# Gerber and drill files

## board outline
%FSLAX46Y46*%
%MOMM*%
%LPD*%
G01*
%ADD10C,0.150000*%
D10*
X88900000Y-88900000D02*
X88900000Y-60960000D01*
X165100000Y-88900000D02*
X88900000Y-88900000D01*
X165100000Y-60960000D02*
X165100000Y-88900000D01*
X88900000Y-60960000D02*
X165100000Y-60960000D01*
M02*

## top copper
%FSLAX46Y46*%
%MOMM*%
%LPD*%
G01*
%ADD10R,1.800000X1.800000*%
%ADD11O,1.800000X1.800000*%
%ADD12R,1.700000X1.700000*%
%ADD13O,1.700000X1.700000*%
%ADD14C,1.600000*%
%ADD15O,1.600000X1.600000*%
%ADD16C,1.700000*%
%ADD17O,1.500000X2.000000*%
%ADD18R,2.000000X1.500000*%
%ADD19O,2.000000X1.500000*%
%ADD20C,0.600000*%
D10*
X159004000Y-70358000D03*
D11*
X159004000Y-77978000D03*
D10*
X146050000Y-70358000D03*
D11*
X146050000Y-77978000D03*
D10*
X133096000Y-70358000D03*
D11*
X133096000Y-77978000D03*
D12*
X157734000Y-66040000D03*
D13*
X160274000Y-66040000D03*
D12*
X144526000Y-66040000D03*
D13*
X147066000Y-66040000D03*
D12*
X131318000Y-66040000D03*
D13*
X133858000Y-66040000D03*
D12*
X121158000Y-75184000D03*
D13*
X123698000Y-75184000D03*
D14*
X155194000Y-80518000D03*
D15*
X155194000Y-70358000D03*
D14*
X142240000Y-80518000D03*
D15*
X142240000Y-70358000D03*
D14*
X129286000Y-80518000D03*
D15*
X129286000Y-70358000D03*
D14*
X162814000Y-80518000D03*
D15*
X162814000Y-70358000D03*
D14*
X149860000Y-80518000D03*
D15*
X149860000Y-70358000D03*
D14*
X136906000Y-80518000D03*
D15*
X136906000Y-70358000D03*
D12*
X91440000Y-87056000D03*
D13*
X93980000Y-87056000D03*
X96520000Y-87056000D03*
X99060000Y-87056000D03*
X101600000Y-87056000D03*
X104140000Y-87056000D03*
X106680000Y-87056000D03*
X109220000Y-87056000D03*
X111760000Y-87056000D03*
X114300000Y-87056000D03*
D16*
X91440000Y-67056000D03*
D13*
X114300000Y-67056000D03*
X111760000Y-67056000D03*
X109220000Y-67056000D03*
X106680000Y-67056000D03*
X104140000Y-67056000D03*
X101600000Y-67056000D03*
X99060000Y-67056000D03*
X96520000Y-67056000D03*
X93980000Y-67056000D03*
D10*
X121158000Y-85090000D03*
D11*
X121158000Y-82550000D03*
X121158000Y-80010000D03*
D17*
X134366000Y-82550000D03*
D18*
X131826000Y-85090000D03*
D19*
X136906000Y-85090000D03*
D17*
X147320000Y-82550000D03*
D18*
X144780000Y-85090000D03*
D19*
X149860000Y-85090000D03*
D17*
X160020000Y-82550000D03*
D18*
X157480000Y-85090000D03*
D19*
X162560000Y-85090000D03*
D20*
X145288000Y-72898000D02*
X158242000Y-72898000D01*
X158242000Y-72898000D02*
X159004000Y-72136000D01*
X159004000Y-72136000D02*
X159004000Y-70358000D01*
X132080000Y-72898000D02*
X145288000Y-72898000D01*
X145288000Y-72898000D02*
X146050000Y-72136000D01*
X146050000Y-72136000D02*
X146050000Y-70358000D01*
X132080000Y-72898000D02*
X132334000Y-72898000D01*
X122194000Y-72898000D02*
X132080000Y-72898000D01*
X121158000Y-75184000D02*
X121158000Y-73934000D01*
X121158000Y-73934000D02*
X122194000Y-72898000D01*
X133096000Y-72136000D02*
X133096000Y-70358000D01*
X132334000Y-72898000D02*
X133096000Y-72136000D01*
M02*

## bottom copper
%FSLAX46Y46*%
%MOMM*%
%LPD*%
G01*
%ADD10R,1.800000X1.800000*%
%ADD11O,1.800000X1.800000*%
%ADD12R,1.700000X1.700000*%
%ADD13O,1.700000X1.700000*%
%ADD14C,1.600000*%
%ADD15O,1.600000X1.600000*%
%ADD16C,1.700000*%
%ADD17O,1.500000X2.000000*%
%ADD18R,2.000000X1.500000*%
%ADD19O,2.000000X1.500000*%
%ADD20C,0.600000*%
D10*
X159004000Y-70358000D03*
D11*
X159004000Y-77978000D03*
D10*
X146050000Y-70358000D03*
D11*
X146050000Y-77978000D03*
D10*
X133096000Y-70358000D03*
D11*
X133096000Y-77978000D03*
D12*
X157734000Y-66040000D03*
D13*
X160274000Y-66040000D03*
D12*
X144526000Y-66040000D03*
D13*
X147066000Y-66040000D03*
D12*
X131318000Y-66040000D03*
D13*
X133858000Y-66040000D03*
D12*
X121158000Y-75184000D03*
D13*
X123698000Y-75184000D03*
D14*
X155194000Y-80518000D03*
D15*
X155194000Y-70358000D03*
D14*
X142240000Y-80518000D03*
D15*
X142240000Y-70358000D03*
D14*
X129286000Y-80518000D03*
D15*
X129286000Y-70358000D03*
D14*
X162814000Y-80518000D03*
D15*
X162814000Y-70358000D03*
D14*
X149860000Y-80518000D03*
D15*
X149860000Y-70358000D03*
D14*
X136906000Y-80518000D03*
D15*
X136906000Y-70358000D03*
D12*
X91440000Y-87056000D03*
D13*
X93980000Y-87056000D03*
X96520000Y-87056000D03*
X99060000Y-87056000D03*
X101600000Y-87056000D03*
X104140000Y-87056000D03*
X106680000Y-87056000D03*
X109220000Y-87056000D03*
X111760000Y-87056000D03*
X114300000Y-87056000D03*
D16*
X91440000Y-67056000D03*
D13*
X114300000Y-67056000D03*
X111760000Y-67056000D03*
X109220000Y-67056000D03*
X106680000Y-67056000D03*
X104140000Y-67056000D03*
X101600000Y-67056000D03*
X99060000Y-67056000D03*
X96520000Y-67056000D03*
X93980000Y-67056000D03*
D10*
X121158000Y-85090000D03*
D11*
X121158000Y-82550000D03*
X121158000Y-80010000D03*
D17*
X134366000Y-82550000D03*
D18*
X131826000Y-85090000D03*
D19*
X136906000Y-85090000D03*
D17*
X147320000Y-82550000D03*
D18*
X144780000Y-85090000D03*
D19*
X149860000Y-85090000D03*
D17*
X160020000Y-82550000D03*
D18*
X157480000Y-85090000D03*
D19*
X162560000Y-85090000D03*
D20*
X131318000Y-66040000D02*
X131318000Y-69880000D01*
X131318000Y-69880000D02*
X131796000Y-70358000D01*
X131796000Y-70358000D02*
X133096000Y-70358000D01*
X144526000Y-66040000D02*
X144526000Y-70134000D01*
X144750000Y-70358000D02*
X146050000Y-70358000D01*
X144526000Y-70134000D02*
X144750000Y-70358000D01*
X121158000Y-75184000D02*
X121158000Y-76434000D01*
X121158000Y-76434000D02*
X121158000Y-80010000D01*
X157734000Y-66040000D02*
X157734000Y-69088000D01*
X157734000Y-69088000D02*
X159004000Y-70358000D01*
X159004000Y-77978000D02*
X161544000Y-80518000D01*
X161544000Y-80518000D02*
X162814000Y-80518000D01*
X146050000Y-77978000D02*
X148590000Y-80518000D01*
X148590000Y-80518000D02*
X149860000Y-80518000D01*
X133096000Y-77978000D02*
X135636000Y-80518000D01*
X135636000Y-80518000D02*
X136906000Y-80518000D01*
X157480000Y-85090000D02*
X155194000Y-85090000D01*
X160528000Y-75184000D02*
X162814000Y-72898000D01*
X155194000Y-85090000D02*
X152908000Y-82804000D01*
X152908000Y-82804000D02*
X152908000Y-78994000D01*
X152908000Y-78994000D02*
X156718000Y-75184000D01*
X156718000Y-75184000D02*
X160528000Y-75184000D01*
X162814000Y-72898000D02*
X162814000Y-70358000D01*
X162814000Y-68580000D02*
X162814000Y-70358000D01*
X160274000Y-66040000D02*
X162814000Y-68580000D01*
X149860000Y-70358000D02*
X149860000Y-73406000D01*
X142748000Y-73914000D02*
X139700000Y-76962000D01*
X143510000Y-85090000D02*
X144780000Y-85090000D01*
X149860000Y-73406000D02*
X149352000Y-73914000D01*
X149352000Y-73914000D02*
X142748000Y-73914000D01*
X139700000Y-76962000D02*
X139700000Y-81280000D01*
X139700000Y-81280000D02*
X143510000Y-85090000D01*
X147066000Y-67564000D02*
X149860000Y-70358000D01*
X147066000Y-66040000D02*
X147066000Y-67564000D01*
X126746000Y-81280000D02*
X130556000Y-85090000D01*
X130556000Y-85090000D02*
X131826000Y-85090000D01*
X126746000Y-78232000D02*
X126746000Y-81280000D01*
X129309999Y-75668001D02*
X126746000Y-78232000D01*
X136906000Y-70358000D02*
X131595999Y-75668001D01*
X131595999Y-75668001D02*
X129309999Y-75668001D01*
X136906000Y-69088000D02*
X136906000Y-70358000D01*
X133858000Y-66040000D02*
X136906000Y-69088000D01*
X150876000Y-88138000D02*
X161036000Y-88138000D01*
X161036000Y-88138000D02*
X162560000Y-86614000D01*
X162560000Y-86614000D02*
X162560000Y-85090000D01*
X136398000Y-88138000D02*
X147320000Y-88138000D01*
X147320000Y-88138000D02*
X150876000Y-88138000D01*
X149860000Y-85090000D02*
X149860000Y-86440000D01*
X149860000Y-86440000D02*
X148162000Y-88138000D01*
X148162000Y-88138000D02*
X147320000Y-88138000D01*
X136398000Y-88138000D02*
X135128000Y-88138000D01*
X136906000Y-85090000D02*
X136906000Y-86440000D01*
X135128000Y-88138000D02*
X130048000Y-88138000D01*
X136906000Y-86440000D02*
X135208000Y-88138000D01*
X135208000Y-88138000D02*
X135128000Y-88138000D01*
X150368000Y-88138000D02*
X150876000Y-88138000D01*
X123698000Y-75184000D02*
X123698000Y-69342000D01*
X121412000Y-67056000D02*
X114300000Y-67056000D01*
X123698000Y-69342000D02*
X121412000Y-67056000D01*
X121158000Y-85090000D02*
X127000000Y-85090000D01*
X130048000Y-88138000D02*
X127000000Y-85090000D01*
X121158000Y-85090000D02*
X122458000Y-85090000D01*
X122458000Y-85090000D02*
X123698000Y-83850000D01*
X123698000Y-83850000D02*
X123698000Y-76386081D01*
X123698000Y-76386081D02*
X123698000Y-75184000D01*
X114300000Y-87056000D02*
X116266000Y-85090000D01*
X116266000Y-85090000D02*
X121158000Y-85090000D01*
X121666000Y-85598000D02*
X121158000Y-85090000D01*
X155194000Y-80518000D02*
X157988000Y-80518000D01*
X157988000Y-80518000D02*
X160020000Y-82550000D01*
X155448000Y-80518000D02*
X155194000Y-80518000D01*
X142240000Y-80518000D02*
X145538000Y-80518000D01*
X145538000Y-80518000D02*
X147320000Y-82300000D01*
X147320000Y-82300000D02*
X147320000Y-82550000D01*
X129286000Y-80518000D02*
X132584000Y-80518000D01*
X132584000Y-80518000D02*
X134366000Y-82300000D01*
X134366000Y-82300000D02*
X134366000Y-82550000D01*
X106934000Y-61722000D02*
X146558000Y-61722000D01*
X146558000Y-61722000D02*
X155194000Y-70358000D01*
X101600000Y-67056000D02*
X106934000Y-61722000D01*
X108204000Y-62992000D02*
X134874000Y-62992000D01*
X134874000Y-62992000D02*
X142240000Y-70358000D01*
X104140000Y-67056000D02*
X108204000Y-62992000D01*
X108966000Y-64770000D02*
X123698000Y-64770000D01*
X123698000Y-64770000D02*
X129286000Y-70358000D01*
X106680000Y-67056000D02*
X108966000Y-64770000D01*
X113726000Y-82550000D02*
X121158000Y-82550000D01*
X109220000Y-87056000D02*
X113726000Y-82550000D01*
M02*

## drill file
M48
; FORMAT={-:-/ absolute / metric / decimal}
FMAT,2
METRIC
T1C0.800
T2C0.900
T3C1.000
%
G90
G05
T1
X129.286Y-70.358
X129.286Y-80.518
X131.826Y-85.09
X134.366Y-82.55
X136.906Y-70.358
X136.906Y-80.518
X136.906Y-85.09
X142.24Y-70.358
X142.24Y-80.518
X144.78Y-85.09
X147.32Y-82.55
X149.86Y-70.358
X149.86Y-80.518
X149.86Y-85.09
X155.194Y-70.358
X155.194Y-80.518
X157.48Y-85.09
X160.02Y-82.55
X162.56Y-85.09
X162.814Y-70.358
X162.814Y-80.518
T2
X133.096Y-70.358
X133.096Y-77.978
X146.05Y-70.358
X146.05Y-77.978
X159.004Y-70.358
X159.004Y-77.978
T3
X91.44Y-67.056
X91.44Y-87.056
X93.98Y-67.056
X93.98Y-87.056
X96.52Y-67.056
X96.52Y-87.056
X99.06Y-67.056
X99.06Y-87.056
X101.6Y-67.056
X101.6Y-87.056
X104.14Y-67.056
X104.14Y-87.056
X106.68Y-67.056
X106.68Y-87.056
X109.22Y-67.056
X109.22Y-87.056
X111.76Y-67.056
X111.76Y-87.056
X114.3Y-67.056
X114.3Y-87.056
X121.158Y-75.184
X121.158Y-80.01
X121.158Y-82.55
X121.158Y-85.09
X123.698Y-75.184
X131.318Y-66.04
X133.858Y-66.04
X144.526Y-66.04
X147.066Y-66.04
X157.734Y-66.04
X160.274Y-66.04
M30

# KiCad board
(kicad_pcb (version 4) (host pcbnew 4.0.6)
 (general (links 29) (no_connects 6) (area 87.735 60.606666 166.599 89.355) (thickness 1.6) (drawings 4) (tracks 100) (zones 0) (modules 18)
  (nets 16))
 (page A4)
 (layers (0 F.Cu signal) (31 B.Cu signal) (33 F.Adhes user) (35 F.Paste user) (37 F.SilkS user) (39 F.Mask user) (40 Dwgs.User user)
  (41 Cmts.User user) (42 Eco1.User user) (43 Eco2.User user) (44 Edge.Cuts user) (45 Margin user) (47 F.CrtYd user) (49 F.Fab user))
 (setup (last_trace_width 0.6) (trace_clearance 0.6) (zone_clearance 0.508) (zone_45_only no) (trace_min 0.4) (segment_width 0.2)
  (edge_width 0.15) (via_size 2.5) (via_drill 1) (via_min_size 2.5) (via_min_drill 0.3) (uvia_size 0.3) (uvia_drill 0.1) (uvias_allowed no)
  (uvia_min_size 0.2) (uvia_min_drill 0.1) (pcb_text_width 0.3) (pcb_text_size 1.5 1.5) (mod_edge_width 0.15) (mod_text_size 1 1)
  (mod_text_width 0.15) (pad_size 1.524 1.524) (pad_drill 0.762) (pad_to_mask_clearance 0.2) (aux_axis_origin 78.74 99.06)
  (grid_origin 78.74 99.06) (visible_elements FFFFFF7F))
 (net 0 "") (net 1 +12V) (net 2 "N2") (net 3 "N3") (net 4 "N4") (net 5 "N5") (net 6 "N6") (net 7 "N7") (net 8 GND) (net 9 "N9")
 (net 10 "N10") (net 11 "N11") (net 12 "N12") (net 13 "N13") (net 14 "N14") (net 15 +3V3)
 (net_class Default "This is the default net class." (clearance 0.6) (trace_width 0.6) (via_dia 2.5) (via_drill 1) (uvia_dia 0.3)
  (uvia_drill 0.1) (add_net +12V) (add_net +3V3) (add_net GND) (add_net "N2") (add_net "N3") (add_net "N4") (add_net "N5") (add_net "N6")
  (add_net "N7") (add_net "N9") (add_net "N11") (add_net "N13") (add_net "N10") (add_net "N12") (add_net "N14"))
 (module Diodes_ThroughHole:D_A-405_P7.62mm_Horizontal (layer F.Cu) (at 159.004 70.358 270)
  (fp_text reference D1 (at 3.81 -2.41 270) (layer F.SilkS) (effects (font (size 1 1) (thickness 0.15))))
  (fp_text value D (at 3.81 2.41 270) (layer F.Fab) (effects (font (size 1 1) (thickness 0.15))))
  (pad 1 thru_hole rect (at 0 0 270) (size 1.8 1.8) (drill 0.9) (layers *.Cu *.Mask) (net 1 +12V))
  (pad 2 thru_hole oval (at 7.62 0 270) (size 1.8 1.8) (drill 0.9) (layers *.Cu *.Mask) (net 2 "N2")))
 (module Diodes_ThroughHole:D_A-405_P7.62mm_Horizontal (layer F.Cu) (at 146.05 70.358 270)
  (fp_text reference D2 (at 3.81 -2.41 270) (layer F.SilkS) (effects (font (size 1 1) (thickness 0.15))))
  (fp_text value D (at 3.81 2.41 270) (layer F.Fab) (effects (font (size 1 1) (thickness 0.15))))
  (pad 1 thru_hole rect (at 0 0 270) (size 1.8 1.8) (drill 0.9) (layers *.Cu *.Mask) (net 1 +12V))
  (pad 2 thru_hole oval (at 7.62 0 270) (size 1.8 1.8) (drill 0.9) (layers *.Cu *.Mask) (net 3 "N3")))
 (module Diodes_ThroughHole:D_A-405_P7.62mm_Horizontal (layer F.Cu) (at 133.096 70.358 270)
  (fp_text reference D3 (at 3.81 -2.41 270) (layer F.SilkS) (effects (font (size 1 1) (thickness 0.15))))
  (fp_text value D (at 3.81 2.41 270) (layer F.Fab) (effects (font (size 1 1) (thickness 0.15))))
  (pad 1 thru_hole rect (at 0 0 270) (size 1.8 1.8) (drill 0.9) (layers *.Cu *.Mask) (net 1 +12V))
  (pad 2 thru_hole oval (at 7.62 0 270) (size 1.8 1.8) (drill 0.9) (layers *.Cu *.Mask) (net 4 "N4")))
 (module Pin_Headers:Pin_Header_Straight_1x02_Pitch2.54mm (layer F.Cu) (at 157.734 66.04 90)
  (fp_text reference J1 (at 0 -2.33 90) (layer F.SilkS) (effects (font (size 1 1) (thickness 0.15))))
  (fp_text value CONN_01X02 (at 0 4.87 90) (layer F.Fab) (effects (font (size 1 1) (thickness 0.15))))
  (pad 1 thru_hole rect (at 0 0 90) (size 1.7 1.7) (drill 1) (layers *.Cu *.Mask) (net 1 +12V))
  (pad 2 thru_hole oval (at 0 2.54 90) (size 1.7 1.7) (drill 1) (layers *.Cu *.Mask) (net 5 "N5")))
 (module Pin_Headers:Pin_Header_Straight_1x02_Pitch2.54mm (layer F.Cu) (at 144.526 66.04 90)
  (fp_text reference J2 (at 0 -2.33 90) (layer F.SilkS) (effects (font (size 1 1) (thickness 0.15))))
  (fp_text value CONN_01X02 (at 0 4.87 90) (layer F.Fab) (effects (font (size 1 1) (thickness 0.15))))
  (pad 1 thru_hole rect (at 0 0 90) (size 1.7 1.7) (drill 1) (layers *.Cu *.Mask) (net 1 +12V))
  (pad 2 thru_hole oval (at 0 2.54 90) (size 1.7 1.7) (drill 1) (layers *.Cu *.Mask) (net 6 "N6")))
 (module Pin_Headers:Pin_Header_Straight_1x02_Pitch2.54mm (layer F.Cu) (at 131.318 66.04 90)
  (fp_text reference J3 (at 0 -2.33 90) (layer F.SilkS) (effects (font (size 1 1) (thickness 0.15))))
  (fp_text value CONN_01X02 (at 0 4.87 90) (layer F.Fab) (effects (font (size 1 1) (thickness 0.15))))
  (pad 1 thru_hole rect (at 0 0 90) (size 1.7 1.7) (drill 1) (layers *.Cu *.Mask) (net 1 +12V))
  (pad 2 thru_hole oval (at 0 2.54 90) (size 1.7 1.7) (drill 1) (layers *.Cu *.Mask) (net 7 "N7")))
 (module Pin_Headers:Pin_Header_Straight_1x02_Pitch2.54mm (layer F.Cu) (at 121.158 75.184 90)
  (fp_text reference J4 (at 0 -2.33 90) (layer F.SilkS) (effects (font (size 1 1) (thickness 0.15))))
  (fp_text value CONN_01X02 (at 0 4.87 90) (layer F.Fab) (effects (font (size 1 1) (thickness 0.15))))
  (pad 1 thru_hole rect (at 0 0 90) (size 1.7 1.7) (drill 1) (layers *.Cu *.Mask) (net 1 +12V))
  (pad 2 thru_hole oval (at 0 2.54 90) (size 1.7 1.7) (drill 1) (layers *.Cu *.Mask) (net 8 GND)))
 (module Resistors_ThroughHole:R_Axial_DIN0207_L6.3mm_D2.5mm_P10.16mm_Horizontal (layer F.Cu) (at 155.194 80.518 90)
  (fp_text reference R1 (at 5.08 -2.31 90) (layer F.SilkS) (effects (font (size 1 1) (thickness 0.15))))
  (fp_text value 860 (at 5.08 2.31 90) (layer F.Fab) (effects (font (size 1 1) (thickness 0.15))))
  (pad 1 thru_hole circle (at 0 0 90) (size 1.6 1.6) (drill 0.8) (layers *.Cu *.Mask) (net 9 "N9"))
  (pad 2 thru_hole oval (at 10.16 0 90) (size 1.6 1.6) (drill 0.8) (layers *.Cu *.Mask) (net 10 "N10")))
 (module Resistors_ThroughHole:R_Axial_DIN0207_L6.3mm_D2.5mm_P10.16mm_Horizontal (layer F.Cu) (at 142.24 80.518 90)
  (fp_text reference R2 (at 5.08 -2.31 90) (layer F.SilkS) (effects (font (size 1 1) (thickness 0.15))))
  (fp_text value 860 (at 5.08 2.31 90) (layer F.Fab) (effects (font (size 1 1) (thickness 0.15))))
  (pad 1 thru_hole circle (at 0 0 90) (size 1.6 1.6) (drill 0.8) (layers *.Cu *.Mask) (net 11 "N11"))
  (pad 2 thru_hole oval (at 10.16 0 90) (size 1.6 1.6) (drill 0.8) (layers *.Cu *.Mask) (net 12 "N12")))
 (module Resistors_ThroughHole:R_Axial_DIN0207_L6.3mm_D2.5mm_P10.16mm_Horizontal (layer F.Cu) (at 129.286 80.518 90)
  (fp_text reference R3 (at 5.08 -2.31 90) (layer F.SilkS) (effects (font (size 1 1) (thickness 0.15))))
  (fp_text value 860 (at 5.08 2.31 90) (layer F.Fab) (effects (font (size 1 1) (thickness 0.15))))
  (pad 1 thru_hole circle (at 0 0 90) (size 1.6 1.6) (drill 0.8) (layers *.Cu *.Mask) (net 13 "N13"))
  (pad 2 thru_hole oval (at 10.16 0 90) (size 1.6 1.6) (drill 0.8) (layers *.Cu *.Mask) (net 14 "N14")))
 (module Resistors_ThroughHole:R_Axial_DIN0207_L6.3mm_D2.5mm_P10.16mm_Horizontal (layer F.Cu) (at 162.814 80.518 90)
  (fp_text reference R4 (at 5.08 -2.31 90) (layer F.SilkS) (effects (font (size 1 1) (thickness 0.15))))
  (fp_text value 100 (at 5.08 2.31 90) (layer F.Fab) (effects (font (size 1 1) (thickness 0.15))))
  (pad 1 thru_hole circle (at 0 0 90) (size 1.6 1.6) (drill 0.8) (layers *.Cu *.Mask) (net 2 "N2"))
  (pad 2 thru_hole oval (at 10.16 0 90) (size 1.6 1.6) (drill 0.8) (layers *.Cu *.Mask) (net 5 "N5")))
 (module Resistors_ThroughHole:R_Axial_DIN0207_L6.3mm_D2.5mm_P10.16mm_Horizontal (layer F.Cu) (at 149.86 80.518 90)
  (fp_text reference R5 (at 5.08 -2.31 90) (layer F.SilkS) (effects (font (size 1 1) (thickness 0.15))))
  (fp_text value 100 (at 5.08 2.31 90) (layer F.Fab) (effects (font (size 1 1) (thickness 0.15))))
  (pad 1 thru_hole circle (at 0 0 90) (size 1.6 1.6) (drill 0.8) (layers *.Cu *.Mask) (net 3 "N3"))
  (pad 2 thru_hole oval (at 10.16 0 90) (size 1.6 1.6) (drill 0.8) (layers *.Cu *.Mask) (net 6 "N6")))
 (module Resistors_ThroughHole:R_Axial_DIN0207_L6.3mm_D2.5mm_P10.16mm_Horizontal (layer F.Cu) (at 136.906 80.518 90)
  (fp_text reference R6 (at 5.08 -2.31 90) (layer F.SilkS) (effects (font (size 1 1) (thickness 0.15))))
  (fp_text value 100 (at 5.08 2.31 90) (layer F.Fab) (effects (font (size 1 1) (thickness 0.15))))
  (pad 1 thru_hole circle (at 0 0 90) (size 1.6 1.6) (drill 0.8) (layers *.Cu *.Mask) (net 4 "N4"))
  (pad 2 thru_hole oval (at 10.16 0 90) (size 1.6 1.6) (drill 0.8) (layers *.Cu *.Mask) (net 7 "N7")))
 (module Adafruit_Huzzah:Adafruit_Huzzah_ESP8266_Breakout (layer F.Cu) (at 91.44 77.056 90)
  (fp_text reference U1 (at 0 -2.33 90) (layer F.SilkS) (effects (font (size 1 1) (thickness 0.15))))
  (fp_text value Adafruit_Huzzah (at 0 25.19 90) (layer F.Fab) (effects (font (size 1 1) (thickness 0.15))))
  (pad 1 thru_hole rect (at -10 0 90) (size 1.7 1.7) (drill 1) (layers *.Cu *.Mask))
  (pad 3 thru_hole oval (at -10 2.54 90) (size 1.7 1.7) (drill 1) (layers *.Cu *.Mask))
  (pad 5 thru_hole oval (at -10 5.08 90) (size 1.7 1.7) (drill 1) (layers *.Cu *.Mask))
  (pad 7 thru_hole oval (at -10 7.62 90) (size 1.7 1.7) (drill 1) (layers *.Cu *.Mask))
  (pad 9 thru_hole oval (at -10 10.16 90) (size 1.7 1.7) (drill 1) (layers *.Cu *.Mask))
  (pad 11 thru_hole oval (at -10 12.7 90) (size 1.7 1.7) (drill 1) (layers *.Cu *.Mask))
  (pad 13 thru_hole oval (at -10 15.24 90) (size 1.7 1.7) (drill 1) (layers *.Cu *.Mask))
  (pad 15 thru_hole oval (at -10 17.78 90) (size 1.7 1.7) (drill 1) (layers *.Cu *.Mask) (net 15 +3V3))
  (pad 17 thru_hole oval (at -10 20.32 90) (size 1.7 1.7) (drill 1) (layers *.Cu *.Mask))
  (pad 19 thru_hole oval (at -10 22.86 90) (size 1.7 1.7) (drill 1) (layers *.Cu *.Mask) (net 8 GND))
  (pad 2 thru_hole circle (at 10 0 90) (size 1.7 1.7) (drill 1) (layers *.Cu *.Mask))
  (pad 20 thru_hole oval (at 10 22.86 90) (size 1.7 1.7) (drill 1) (layers *.Cu *.Mask) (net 8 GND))
  (pad 18 thru_hole oval (at 10 20.32 90) (size 1.7 1.7) (drill 1) (layers *.Cu *.Mask))
  (pad 16 thru_hole oval (at 10 17.78 90) (size 1.7 1.7) (drill 1) (layers *.Cu *.Mask))
  (pad 14 thru_hole oval (at 10 15.24 90) (size 1.7 1.7) (drill 1) (layers *.Cu *.Mask) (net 14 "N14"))
  (pad 12 thru_hole oval (at 10 12.7 90) (size 1.7 1.7) (drill 1) (layers *.Cu *.Mask) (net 12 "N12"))
  (pad 10 thru_hole oval (at 10 10.16 90) (size 1.7 1.7) (drill 1) (layers *.Cu *.Mask) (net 10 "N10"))
  (pad 8 thru_hole oval (at 10 7.62 90) (size 1.7 1.7) (drill 1) (layers *.Cu *.Mask))
  (pad 6 thru_hole oval (at 10 5.08 90) (size 1.7 1.7) (drill 1) (layers *.Cu *.Mask))
  (pad 4 thru_hole oval (at 10 2.54 90) (size 1.7 1.7) (drill 1) (layers *.Cu *.Mask)))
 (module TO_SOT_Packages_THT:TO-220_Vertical (layer F.Cu) (at 121.158 85.09 90)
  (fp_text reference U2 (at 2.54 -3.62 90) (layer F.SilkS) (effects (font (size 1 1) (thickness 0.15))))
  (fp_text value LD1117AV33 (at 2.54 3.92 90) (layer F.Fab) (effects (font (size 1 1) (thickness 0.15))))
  (pad 1 thru_hole rect (at 0 0 90) (size 1.8 1.8) (drill 1) (layers *.Cu *.Mask) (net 8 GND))
  (pad 2 thru_hole oval (at 2.54 0 90) (size 1.8 1.8) (drill 1) (layers *.Cu *.Mask) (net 15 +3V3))
  (pad 3 thru_hole oval (at 5.08 0 90) (size 1.8 1.8) (drill 1) (layers *.Cu *.Mask) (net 1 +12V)))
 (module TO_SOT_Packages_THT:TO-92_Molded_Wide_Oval (layer F.Cu) (at 131.826 85.09)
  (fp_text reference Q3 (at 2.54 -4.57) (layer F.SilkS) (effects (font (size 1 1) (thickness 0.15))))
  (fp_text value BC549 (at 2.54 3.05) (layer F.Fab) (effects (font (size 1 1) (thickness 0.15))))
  (pad 2 thru_hole oval (at 2.54 -2.54 90) (size 2 1.5) (drill 0.8) (layers *.Cu *.Mask) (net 13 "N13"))
  (pad 1 thru_hole rect (at 0 0 90) (size 1.5 2) (drill 0.8) (layers *.Cu *.Mask) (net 7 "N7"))
  (pad 3 thru_hole oval (at 5.08 0 90) (size 1.5 2) (drill 0.8) (layers *.Cu *.Mask) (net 8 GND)))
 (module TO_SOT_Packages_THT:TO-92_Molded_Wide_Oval (layer F.Cu) (at 144.78 85.09)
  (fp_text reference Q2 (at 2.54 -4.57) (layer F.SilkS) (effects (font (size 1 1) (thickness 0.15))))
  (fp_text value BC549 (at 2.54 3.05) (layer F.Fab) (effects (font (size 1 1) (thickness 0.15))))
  (pad 2 thru_hole oval (at 2.54 -2.54 90) (size 2 1.5) (drill 0.8) (layers *.Cu *.Mask) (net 11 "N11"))
  (pad 1 thru_hole rect (at 0 0 90) (size 1.5 2) (drill 0.8) (layers *.Cu *.Mask) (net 6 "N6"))
  (pad 3 thru_hole oval (at 5.08 0 90) (size 1.5 2) (drill 0.8) (layers *.Cu *.Mask) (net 8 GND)))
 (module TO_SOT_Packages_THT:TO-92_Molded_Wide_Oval (layer F.Cu) (at 157.48 85.09)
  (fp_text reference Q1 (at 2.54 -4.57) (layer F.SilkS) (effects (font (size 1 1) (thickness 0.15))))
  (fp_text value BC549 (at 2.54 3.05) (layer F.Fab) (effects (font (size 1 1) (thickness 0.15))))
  (pad 2 thru_hole oval (at 2.54 -2.54 90) (size 2 1.5) (drill 0.8) (layers *.Cu *.Mask) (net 9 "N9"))
  (pad 1 thru_hole rect (at 0 0 90) (size 1.5 2) (drill 0.8) (layers *.Cu *.Mask) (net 5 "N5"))
  (pad 3 thru_hole oval (at 5.08 0 90) (size 1.5 2) (drill 0.8) (layers *.Cu *.Mask) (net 8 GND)))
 (gr_line (start 88.9 88.9) (end 88.9 60.96) (layer Edge.Cuts) (width 0.15))
 (gr_line (start 165.1 88.9) (end 88.9 88.9) (layer Edge.Cuts) (width 0.15))
 (gr_line (start 165.1 60.96) (end 165.1 88.9) (layer Edge.Cuts) (width 0.15))
 (gr_line (start 88.9 60.96) (end 165.1 60.96) (layer Edge.Cuts) (width 0.15))
 (segment (start 145.288 72.898) (end 158.242 72.898) (width 0.6) (layer F.Cu) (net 1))
 (segment (start 158.242 72.898) (end 159.004 72.136) (width 0.6) (layer F.Cu) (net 1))
 (segment (start 159.004 72.136) (end 159.004 70.358) (width 0.6) (layer F.Cu) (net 1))
 (segment (start 132.08 72.898) (end 145.288 72.898) (width 0.6) (layer F.Cu) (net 1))
 (segment (start 145.288 72.898) (end 146.05 72.136) (width 0.6) (layer F.Cu) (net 1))
 (segment (start 146.05 72.136) (end 146.05 70.358) (width 0.6) (layer F.Cu) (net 1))
 (segment (start 132.08 72.898) (end 132.334 72.898) (width 0.6) (layer F.Cu) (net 1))
 (segment (start 122.194 72.898) (end 132.08 72.898) (width 0.6) (layer F.Cu) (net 1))
 (segment (start 121.158 75.184) (end 121.158 73.934) (width 0.6) (layer F.Cu) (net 1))
 (segment (start 121.158 73.934) (end 122.194 72.898) (width 0.6) (layer F.Cu) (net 1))
 (segment (start 133.096 72.136) (end 133.096 70.358) (width 0.6) (layer F.Cu) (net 1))
 (segment (start 132.334 72.898) (end 133.096 72.136) (width 0.6) (layer F.Cu) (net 1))
 (segment (start 131.318 66.04) (end 131.318 69.88) (width 0.6) (layer B.Cu) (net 1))
 (segment (start 131.318 69.88) (end 131.796 70.358) (width 0.6) (layer B.Cu) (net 1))
 (segment (start 131.796 70.358) (end 133.096 70.358) (width 0.6) (layer B.Cu) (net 1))
 (segment (start 144.526 66.04) (end 144.526 70.134) (width 0.6) (layer B.Cu) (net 1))
 (segment (start 144.75 70.358) (end 146.05 70.358) (width 0.6) (layer B.Cu) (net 1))
 (segment (start 144.526 70.134) (end 144.75 70.358) (width 0.6) (layer B.Cu) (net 1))
 (segment (start 121.158 75.184) (end 121.158 76.434) (width 0.6) (layer B.Cu) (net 1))
 (segment (start 121.158 76.434) (end 121.158 80.01) (width 0.6) (layer B.Cu) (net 1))
 (segment (start 157.734 66.04) (end 157.734 69.088) (width 0.6) (layer B.Cu) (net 1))
 (segment (start 157.734 69.088) (end 159.004 70.358) (width 0.6) (layer B.Cu) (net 1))
 (segment (start 159.004 77.978) (end 161.544 80.518) (width 0.6) (layer B.Cu) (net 2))
 (segment (start 161.544 80.518) (end 162.814 80.518) (width 0.6) (layer B.Cu) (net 2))
 (segment (start 146.05 77.978) (end 148.59 80.518) (width 0.6) (layer B.Cu) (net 3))
 (segment (start 148.59 80.518) (end 149.86 80.518) (width 0.6) (layer B.Cu) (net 3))
 (segment (start 133.096 77.978) (end 135.636 80.518) (width 0.6) (layer B.Cu) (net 4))
 (segment (start 135.636 80.518) (end 136.906 80.518) (width 0.6) (layer B.Cu) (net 4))
 (segment (start 157.48 85.09) (end 155.194 85.09) (width 0.6) (layer B.Cu) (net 5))
 (segment (start 160.528 75.184) (end 162.814 72.898) (width 0.6) (layer B.Cu) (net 5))
 (segment (start 155.194 85.09) (end 152.908 82.804) (width 0.6) (layer B.Cu) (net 5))
 (segment (start 152.908 82.804) (end 152.908 78.994) (width 0.6) (layer B.Cu) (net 5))
 (segment (start 152.908 78.994) (end 156.718 75.184) (width 0.6) (layer B.Cu) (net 5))
 (segment (start 156.718 75.184) (end 160.528 75.184) (width 0.6) (layer B.Cu) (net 5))
 (segment (start 162.814 72.898) (end 162.814 70.358) (width 0.6) (layer B.Cu) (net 5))
 (segment (start 162.814 68.58) (end 162.814 70.358) (width 0.6) (layer B.Cu) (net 5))
 (segment (start 160.274 66.04) (end 162.814 68.58) (width 0.6) (layer B.Cu) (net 5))
 (segment (start 149.86 70.358) (end 149.86 73.406) (width 0.6) (layer B.Cu) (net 6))
 (segment (start 142.748 73.914) (end 139.7 76.962) (width 0.6) (layer B.Cu) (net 6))
 (segment (start 143.51 85.09) (end 144.78 85.09) (width 0.6) (layer B.Cu) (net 6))
 (segment (start 149.86 73.406) (end 149.352 73.914) (width 0.6) (layer B.Cu) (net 6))
 (segment (start 149.352 73.914) (end 142.748 73.914) (width 0.6) (layer B.Cu) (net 6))
 (segment (start 139.7 76.962) (end 139.7 81.28) (width 0.6) (layer B.Cu) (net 6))
 (segment (start 139.7 81.28) (end 143.51 85.09) (width 0.6) (layer B.Cu) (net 6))
 (segment (start 147.066 67.564) (end 149.86 70.358) (width 0.6) (layer B.Cu) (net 6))
 (segment (start 147.066 66.04) (end 147.066 67.564) (width 0.6) (layer B.Cu) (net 6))
 (segment (start 126.746 81.28) (end 130.556 85.09) (width 0.6) (layer B.Cu) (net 7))
 (segment (start 130.556 85.09) (end 131.826 85.09) (width 0.6) (layer B.Cu) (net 7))
 (segment (start 126.746 78.232) (end 126.746 81.28) (width 0.6) (layer B.Cu) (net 7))
 (segment (start 129.309999 75.668001) (end 126.746 78.232) (width 0.6) (layer B.Cu) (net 7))
 (segment (start 136.906 70.358) (end 131.595999 75.668001) (width 0.6) (layer B.Cu) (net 7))
 (segment (start 131.595999 75.668001) (end 129.309999 75.668001) (width 0.6) (layer B.Cu) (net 7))
 (segment (start 136.906 69.088) (end 136.906 70.358) (width 0.6) (layer B.Cu) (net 7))
 (segment (start 133.858 66.04) (end 136.906 69.088) (width 0.6) (layer B.Cu) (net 7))
 (segment (start 150.876 88.138) (end 161.036 88.138) (width 0.6) (layer B.Cu) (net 8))
 (segment (start 161.036 88.138) (end 162.56 86.614) (width 0.6) (layer B.Cu) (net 8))
 (segment (start 162.56 86.614) (end 162.56 85.09) (width 0.6) (layer B.Cu) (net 8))
 (segment (start 136.398 88.138) (end 147.32 88.138) (width 0.6) (layer B.Cu) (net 8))
 (segment (start 147.32 88.138) (end 150.876 88.138) (width 0.6) (layer B.Cu) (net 8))
 (segment (start 149.86 85.09) (end 149.86 86.44) (width 0.6) (layer B.Cu) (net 8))
 (segment (start 149.86 86.44) (end 148.162 88.138) (width 0.6) (layer B.Cu) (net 8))
 (segment (start 148.162 88.138) (end 147.32 88.138) (width 0.6) (layer B.Cu) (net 8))
 (segment (start 136.398 88.138) (end 135.128 88.138) (width 0.6) (layer B.Cu) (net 8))
 (segment (start 136.906 85.09) (end 136.906 86.44) (width 0.6) (layer B.Cu) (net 8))
 (segment (start 135.128 88.138) (end 130.048 88.138) (width 0.6) (layer B.Cu) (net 8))
 (segment (start 136.906 86.44) (end 135.208 88.138) (width 0.6) (layer B.Cu) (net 8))
 (segment (start 135.208 88.138) (end 135.128 88.138) (width 0.6) (layer B.Cu) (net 8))
 (segment (start 150.368 88.138) (end 150.876 88.138) (width 0.6) (layer B.Cu) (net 8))
 (segment (start 123.698 75.184) (end 123.698 69.342) (width 0.6) (layer B.Cu) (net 8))
 (segment (start 121.412 67.056) (end 114.3 67.056) (width 0.6) (layer B.Cu) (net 8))
 (segment (start 123.698 69.342) (end 121.412 67.056) (width 0.6) (layer B.Cu) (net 8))
 (segment (start 121.158 85.09) (end 127 85.09) (width 0.6) (layer B.Cu) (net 8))
 (segment (start 130.048 88.138) (end 127 85.09) (width 0.6) (layer B.Cu) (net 8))
 (segment (start 121.158 85.09) (end 122.458 85.09) (width 0.6) (layer B.Cu) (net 8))
 (segment (start 122.458 85.09) (end 123.698 83.85) (width 0.6) (layer B.Cu) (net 8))
 (segment (start 123.698 83.85) (end 123.698 76.386081) (width 0.6) (layer B.Cu) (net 8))
 (segment (start 123.698 76.386081) (end 123.698 75.184) (width 0.6) (layer B.Cu) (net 8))
 (segment (start 114.3 87.056) (end 116.266 85.09) (width 0.6) (layer B.Cu) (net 8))
 (segment (start 116.266 85.09) (end 121.158 85.09) (width 0.6) (layer B.Cu) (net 8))
 (segment (start 121.666 85.598) (end 121.158 85.09) (width 0.6) (layer B.Cu) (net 8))
 (segment (start 155.194 80.518) (end 157.988 80.518) (width 0.6) (layer B.Cu) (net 9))
 (segment (start 157.988 80.518) (end 160.02 82.55) (width 0.6) (layer B.Cu) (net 9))
 (segment (start 155.448 80.518) (end 155.194 80.518) (width 0.6) (layer B.Cu) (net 9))
 (segment (start 142.24 80.518) (end 145.538 80.518) (width 0.6) (layer B.Cu) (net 11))
 (segment (start 145.538 80.518) (end 147.32 82.3) (width 0.6) (layer B.Cu) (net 11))
 (segment (start 147.32 82.3) (end 147.32 82.55) (width 0.6) (layer B.Cu) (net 11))
 (segment (start 129.286 80.518) (end 132.584 80.518) (width 0.6) (layer B.Cu) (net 13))
 (segment (start 132.584 80.518) (end 134.366 82.3) (width 0.6) (layer B.Cu) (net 13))
 (segment (start 134.366 82.3) (end 134.366 82.55) (width 0.6) (layer B.Cu) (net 13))
 (segment (start 106.934 61.722) (end 146.558 61.722) (width 0.6) (layer B.Cu) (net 10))
 (segment (start 146.558 61.722) (end 155.194 70.358) (width 0.6) (layer B.Cu) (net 10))
 (segment (start 101.6 67.056) (end 106.934 61.722) (width 0.6) (layer B.Cu) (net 10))
 (segment (start 108.204 62.992) (end 134.874 62.992) (width 0.6) (layer B.Cu) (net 12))
 (segment (start 134.874 62.992) (end 142.24 70.358) (width 0.6) (layer B.Cu) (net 12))
 (segment (start 104.14 67.056) (end 108.204 62.992) (width 0.6) (layer B.Cu) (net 12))
 (segment (start 108.966 64.77) (end 123.698 64.77) (width 0.6) (layer B.Cu) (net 14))
 (segment (start 123.698 64.77) (end 129.286 70.358) (width 0.6) (layer B.Cu) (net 14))
 (segment (start 106.68 67.056) (end 108.966 64.77) (width 0.6) (layer B.Cu) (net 14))
 (segment (start 113.726 82.55) (end 121.158 82.55) (width 0.6) (layer B.Cu) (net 15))
 (segment (start 109.22 87.056) (end 113.726 82.55) (width 0.6) (layer B.Cu) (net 15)))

